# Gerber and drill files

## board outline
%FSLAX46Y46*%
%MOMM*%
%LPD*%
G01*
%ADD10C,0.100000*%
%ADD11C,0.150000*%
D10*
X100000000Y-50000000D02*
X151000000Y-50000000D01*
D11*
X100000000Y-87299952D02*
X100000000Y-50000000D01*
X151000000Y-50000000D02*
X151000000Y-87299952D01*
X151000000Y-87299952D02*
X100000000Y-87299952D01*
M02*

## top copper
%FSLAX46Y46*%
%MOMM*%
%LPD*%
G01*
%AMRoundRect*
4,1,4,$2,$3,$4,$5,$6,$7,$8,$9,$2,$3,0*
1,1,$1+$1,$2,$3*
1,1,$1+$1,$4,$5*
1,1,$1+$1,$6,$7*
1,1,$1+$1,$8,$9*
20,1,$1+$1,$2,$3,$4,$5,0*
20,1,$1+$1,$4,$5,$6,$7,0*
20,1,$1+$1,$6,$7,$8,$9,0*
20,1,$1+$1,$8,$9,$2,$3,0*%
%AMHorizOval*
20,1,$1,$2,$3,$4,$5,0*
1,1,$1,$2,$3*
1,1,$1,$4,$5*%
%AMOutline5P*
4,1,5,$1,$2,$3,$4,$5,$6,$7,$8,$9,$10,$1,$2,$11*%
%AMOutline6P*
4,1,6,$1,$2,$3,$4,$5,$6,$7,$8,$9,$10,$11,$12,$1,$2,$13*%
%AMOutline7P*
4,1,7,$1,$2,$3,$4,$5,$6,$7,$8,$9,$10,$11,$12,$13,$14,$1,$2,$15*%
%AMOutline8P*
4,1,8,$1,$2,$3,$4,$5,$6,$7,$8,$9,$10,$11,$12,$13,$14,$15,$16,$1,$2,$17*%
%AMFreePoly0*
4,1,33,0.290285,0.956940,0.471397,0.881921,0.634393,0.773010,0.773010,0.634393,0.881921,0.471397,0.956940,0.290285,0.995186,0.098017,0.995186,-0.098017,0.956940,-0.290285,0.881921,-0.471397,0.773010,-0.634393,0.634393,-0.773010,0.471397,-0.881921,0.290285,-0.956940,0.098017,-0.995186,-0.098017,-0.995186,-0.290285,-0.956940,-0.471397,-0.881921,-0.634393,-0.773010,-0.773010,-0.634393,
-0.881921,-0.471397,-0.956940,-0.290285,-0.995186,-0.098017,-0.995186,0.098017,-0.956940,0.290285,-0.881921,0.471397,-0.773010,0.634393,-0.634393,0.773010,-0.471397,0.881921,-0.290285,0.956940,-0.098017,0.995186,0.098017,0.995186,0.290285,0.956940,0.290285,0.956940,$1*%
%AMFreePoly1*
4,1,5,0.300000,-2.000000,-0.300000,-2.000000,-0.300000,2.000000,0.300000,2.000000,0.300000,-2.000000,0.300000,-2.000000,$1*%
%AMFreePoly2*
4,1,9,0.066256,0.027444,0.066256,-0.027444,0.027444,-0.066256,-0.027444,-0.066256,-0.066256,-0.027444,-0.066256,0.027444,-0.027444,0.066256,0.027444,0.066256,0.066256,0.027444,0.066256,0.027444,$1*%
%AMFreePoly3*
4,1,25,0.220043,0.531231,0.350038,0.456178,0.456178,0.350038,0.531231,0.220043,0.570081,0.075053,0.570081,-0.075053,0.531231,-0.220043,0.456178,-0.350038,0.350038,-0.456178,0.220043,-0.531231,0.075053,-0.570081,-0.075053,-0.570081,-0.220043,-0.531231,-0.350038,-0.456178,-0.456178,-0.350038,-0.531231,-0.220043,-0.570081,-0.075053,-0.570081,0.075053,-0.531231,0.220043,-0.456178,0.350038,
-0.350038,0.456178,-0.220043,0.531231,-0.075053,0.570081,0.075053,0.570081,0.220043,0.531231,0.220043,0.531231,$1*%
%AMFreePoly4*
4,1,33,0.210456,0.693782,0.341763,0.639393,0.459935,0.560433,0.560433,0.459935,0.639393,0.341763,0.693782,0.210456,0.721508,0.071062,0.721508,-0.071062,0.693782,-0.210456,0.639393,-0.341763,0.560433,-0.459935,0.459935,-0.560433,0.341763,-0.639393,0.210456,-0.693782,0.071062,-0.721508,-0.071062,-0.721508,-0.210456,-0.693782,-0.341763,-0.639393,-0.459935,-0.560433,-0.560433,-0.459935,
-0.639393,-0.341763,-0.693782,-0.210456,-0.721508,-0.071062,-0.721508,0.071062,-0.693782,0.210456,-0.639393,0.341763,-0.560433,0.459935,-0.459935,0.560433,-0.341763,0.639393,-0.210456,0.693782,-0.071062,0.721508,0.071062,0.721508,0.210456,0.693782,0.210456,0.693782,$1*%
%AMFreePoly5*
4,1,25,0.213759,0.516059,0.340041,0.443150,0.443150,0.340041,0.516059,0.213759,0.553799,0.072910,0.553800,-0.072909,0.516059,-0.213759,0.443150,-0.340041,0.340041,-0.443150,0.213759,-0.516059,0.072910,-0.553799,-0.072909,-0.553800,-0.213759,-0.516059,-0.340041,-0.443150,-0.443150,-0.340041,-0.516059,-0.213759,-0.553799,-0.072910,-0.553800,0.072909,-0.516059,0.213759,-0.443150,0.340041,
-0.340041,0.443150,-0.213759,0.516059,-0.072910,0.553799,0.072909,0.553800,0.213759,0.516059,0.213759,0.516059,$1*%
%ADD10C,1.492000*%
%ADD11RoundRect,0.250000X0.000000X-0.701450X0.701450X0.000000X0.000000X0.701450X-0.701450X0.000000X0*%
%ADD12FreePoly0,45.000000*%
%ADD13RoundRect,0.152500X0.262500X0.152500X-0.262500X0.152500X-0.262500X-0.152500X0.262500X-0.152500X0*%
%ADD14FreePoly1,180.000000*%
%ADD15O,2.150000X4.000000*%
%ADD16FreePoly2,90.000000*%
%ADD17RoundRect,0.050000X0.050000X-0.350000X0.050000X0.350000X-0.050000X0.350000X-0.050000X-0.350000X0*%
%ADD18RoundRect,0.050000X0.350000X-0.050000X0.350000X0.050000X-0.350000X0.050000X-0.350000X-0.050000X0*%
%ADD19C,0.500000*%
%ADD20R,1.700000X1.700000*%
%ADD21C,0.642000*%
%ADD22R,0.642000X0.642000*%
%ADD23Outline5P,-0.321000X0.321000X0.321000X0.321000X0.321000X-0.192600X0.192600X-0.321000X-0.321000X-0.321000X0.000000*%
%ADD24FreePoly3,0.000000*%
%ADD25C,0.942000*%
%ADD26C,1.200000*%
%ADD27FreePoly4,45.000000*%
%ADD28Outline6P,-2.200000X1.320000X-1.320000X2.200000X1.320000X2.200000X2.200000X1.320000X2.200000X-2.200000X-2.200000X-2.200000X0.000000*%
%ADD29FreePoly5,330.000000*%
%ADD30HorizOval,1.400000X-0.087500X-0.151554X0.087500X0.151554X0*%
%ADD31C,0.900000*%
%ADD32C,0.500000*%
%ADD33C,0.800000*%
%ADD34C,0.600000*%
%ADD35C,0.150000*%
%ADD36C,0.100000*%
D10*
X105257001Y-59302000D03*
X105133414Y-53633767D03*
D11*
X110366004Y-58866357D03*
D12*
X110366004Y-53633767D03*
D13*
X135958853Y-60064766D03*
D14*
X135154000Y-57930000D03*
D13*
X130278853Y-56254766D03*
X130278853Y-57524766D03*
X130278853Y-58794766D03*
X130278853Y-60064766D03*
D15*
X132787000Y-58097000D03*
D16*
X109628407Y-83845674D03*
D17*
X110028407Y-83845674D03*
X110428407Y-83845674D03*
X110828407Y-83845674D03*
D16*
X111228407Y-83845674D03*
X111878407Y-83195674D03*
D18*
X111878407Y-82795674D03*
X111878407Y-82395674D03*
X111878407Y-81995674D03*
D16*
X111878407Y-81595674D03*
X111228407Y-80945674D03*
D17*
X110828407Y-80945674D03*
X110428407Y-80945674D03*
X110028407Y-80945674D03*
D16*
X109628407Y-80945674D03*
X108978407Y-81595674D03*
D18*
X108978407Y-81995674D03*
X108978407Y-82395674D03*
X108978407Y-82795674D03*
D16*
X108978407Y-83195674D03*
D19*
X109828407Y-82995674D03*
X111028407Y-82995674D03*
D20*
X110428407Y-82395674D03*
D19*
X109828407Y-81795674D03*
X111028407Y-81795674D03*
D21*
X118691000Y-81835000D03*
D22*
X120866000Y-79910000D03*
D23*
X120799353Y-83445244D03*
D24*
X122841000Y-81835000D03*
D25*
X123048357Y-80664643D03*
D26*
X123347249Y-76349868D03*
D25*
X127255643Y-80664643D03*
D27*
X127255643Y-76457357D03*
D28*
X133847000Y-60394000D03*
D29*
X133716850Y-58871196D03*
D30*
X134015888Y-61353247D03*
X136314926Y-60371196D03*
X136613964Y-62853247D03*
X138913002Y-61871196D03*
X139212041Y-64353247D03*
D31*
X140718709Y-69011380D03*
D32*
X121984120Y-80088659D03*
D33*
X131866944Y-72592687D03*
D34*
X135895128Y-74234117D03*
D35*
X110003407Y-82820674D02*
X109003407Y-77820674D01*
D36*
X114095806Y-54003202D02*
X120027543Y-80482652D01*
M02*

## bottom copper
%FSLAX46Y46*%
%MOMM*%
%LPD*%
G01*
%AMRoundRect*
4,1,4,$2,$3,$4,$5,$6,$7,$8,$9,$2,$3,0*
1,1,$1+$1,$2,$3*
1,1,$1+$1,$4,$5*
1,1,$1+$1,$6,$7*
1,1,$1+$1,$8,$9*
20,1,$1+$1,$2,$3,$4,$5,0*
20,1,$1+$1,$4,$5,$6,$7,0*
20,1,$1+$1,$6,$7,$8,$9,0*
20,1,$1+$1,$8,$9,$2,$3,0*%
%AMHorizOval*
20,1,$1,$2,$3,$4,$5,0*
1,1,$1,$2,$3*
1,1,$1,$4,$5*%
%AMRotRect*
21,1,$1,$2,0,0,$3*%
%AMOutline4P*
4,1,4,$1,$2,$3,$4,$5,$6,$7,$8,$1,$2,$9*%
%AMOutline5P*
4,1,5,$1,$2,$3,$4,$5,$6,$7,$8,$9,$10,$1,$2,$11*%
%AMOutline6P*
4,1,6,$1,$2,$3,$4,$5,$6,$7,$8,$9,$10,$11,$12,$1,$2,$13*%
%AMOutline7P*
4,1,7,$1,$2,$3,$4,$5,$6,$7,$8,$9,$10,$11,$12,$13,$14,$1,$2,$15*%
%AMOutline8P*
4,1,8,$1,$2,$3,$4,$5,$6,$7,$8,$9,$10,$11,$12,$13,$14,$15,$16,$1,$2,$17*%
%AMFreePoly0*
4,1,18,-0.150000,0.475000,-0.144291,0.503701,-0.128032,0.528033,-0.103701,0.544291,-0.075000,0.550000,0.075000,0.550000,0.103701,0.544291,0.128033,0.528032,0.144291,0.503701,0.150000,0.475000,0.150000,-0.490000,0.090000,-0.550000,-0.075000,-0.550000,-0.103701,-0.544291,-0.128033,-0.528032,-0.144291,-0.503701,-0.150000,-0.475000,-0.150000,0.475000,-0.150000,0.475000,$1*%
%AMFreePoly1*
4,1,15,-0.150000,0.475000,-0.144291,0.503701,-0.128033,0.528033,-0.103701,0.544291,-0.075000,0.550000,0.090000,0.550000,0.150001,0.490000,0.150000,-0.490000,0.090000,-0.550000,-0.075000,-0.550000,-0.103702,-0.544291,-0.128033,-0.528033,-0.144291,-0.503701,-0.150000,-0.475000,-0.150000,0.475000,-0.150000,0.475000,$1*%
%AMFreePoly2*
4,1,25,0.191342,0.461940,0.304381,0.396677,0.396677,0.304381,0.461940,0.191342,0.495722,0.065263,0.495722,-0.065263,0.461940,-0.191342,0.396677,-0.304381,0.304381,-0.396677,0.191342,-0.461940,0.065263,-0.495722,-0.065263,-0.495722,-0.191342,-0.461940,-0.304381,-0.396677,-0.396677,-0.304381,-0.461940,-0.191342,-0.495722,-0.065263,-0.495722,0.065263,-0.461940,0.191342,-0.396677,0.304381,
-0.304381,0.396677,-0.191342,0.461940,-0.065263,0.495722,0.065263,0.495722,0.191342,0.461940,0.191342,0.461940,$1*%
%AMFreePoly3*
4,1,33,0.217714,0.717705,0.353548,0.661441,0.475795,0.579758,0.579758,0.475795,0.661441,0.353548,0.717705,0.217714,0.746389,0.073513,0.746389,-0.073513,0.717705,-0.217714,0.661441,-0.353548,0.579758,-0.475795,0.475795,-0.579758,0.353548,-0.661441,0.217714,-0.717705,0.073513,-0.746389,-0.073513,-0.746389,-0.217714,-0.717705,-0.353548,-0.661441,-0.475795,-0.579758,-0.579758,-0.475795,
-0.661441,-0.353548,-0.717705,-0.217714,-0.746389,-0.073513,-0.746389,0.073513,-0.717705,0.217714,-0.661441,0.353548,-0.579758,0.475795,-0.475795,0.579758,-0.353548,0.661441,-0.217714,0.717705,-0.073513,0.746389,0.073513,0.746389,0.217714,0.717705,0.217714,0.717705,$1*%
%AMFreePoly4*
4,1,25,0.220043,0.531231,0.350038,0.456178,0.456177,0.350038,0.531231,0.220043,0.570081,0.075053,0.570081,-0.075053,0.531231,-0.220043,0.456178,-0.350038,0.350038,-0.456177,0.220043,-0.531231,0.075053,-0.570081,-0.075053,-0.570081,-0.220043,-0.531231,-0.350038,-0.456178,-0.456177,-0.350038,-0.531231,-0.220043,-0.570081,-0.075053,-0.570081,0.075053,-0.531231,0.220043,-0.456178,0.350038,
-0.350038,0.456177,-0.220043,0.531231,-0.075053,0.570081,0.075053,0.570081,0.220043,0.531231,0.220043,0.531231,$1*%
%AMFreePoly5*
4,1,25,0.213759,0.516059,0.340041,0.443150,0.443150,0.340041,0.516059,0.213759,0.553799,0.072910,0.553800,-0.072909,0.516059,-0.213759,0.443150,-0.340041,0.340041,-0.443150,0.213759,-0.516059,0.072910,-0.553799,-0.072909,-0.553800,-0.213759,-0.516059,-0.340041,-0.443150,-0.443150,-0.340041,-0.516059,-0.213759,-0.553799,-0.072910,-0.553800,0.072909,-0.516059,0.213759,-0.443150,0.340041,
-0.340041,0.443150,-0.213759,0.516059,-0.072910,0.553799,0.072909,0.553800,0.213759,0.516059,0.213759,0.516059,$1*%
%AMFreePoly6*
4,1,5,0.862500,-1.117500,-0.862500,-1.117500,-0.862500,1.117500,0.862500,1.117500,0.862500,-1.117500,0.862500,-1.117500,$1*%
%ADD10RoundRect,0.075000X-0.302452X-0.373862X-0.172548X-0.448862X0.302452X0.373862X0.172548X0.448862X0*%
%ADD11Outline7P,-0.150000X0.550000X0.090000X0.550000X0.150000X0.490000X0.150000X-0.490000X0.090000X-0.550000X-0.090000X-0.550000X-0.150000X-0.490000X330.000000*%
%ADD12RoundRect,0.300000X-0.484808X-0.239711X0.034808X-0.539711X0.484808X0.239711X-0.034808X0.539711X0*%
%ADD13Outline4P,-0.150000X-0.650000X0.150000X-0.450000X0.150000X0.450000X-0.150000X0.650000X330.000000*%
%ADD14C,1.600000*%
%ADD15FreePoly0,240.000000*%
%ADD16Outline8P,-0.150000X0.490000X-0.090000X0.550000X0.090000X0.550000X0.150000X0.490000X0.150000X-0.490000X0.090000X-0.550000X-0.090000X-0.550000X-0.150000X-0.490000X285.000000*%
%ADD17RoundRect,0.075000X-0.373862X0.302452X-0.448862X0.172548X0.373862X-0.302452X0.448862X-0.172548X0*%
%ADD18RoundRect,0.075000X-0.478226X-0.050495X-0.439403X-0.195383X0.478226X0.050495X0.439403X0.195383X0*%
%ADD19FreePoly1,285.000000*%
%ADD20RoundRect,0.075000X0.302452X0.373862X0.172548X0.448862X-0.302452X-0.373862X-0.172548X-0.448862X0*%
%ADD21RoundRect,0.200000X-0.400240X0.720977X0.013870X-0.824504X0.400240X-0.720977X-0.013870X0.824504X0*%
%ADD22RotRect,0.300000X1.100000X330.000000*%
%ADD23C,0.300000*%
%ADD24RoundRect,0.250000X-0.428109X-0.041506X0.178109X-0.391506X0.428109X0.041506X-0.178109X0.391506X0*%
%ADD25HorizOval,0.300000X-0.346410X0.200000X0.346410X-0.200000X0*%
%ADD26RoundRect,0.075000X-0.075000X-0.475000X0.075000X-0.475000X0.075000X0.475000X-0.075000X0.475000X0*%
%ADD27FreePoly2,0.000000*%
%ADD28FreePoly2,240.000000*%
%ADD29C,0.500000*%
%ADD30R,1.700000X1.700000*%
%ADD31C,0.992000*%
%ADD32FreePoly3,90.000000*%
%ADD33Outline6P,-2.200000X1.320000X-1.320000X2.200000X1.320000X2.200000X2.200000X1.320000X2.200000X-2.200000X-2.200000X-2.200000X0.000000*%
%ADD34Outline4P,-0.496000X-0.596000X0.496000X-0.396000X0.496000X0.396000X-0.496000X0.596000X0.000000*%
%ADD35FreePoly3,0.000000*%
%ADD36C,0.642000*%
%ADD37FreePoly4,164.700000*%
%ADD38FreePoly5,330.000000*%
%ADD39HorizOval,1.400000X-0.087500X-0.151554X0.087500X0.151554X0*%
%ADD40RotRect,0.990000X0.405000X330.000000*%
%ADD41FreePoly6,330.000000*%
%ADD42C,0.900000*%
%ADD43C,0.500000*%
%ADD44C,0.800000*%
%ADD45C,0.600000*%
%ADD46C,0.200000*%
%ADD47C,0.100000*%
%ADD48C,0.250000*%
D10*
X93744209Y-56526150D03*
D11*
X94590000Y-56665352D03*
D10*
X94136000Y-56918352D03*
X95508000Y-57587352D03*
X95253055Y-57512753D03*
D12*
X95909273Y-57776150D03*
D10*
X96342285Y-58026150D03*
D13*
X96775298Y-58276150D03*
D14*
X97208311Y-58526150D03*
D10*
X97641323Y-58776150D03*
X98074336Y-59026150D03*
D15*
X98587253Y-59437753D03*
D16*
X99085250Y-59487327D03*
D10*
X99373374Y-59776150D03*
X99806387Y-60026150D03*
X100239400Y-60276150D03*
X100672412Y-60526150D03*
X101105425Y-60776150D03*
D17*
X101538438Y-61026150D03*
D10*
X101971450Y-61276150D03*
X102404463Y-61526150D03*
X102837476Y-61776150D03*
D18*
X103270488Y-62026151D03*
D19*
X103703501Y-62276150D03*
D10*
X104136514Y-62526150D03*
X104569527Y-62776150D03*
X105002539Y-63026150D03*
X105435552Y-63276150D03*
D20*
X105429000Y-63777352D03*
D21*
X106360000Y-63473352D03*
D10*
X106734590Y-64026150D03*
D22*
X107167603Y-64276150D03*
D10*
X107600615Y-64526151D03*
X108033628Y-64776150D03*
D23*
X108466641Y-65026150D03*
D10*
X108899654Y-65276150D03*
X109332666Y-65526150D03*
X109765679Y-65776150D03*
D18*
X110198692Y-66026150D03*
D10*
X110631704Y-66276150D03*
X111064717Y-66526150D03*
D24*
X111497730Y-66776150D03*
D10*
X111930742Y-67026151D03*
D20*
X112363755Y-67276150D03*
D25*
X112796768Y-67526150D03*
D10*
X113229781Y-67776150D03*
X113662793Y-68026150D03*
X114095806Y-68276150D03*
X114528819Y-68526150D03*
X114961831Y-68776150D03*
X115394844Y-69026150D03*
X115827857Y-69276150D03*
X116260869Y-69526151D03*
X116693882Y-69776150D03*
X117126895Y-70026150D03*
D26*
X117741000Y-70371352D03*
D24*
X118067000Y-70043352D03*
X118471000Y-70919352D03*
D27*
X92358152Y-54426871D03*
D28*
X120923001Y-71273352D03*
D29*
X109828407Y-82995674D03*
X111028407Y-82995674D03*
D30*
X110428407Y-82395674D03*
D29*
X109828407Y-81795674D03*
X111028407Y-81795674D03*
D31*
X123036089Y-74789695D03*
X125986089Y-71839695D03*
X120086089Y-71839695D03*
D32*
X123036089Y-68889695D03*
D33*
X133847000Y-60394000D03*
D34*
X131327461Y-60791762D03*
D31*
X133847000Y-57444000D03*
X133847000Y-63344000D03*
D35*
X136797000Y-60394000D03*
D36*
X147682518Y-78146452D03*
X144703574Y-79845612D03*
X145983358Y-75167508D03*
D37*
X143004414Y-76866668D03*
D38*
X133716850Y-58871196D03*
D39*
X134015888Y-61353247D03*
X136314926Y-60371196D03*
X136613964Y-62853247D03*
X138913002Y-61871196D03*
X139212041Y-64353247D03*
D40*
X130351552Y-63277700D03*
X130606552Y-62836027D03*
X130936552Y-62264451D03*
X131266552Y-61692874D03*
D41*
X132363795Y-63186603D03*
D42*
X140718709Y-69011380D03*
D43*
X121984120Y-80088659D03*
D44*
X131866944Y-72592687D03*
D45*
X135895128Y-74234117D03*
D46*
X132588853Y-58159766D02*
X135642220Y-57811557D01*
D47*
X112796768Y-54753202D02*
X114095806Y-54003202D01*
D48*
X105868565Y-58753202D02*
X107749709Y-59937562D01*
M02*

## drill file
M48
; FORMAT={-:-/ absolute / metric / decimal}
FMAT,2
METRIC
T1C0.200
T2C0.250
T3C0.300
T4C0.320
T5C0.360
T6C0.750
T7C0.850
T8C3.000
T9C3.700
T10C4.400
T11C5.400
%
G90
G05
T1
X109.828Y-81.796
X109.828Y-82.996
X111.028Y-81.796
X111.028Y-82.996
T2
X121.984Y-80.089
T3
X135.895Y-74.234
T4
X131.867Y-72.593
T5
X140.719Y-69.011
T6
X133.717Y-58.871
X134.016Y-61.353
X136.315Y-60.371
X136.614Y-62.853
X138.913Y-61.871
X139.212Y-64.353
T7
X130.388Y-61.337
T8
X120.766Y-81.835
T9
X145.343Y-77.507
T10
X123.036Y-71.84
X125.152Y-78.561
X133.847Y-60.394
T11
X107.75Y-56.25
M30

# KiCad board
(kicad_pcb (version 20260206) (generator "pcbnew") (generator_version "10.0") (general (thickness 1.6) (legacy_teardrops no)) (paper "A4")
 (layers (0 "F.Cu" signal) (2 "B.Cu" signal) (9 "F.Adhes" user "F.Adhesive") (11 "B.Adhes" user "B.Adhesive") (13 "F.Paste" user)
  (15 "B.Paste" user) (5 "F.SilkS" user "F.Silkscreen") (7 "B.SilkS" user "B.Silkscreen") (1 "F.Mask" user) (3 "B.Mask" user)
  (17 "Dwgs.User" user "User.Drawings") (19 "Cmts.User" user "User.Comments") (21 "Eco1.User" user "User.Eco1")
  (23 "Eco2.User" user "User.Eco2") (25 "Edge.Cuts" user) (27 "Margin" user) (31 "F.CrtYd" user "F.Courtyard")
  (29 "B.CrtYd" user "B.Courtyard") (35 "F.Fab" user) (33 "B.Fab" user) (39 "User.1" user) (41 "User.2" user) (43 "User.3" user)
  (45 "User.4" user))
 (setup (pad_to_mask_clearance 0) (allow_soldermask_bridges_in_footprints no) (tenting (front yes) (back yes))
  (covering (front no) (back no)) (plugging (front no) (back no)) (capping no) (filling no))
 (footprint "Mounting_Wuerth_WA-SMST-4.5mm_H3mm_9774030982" (layer "F.Cu") (at 107.749709 56.250062 45)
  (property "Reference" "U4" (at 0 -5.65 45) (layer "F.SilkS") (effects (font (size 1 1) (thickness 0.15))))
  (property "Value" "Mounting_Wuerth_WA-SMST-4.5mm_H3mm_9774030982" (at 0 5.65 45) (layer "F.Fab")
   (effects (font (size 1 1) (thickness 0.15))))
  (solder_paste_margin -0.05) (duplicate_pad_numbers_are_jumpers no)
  (pad "" smd custom (at -2.607456 -2.607456 15) (size 0.9475 0.9475) (layers) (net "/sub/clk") (clearance 0.1) (zone_connect 0)
   (options (clearance outline) (anchor circle)) (primitives))
  (pad "" smd custom (at -2.222894 2.681511 90) (size 0.8 0.8) (layers "F.Paste") (options (clearance outline) (anchor circle)) (primitives))
  (pad "" np_thru_hole circle (at 0 0 90) (size 5.4 5.4) (drill 5.4) (layers "*.Cu" "*.Mask") (solder_mask_margin 0.05) (clearance 0.2))
  (pad "" smd custom (at 2.607456 -2.607456 135) (size 0.9475 0.9475) (drill (offset -0.2 -0.1)) (layers "F.Paste") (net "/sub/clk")
   (thermal_bridge_angle 30) (options (clearance outline) (anchor circle)) (primitives))
  (pad "" smd custom (at 2.607456 2.607456 45) (size 0.9475 0.9475) (layers "F.Paste") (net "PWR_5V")
   (options (clearance outline) (anchor circle)) (primitives))
  (pad "1" smd circle (at -3.920657 0.395435 45) (size 1.492 1.492) (layers "F.Cu"))
  (pad "1" smd circle (at 0 -3.7 45) (size 1.492 1.492) (layers "F.Cu") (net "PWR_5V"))
  (pad "A1" smd roundrect (at 0 3.7 45) (size 1.492 1.492) (layers "F.Cu") (roundrect_rratio 0.16756))
  (pad "1" smd custom (at 3.7 0 45) (size 2 2) (layers "F.Cu" "F.Mask") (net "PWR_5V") (clearance 0.1) (thermal_gap 0.3)
   (options (clearance outline) (anchor circle)) (primitives)))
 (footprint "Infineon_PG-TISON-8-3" (layer "F.Cu") (at 133.118853 58.159766 180)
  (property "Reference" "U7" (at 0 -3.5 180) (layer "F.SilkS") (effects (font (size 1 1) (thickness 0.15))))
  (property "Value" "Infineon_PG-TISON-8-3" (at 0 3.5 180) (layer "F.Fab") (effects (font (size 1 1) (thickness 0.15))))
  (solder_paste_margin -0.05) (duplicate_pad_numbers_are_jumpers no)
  (pad "" smd rect (at -2.84 -0.635 180) (size 0.73 0.51) (layers "F.Paste"))
  (pad "" smd rect (at -2.84 0.635 180) (size 0.73 0.51) (layers "B.Mask" "F.SilkS") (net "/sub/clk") (clearance 0.1) (thermal_gap 0.3))
  (pad "" smd rect (at -2.84 1.905 180) (size 0.73 0.51) (layers "F.Paste") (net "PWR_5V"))
  (pad "" smd rect (at -1.82 -0.64 180) (size 0.9 0.5) (layers "F.Paste"))
  (pad "" smd rect (at -1.82 0.06 180) (size 0.9 0.5) (layers "F.Paste") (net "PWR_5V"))
  (pad "" smd rect (at -1.647147 0.676766 180) (size 1.2 1.5) (layers "F.Paste") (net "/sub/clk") (clearance 0.1) (thermal_gap 0.5))
  (pad "" smd rect (at -1.82 1.46 180) (size 0.9 0.5) (layers "F.Paste") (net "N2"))
  (pad "" smd rect (at -1.545 -1.6 225) (size 0.35 0.6) (layers "F.Paste") (solder_mask_margin 0.05) (solder_paste_margin -0.03)
   (thermal_bridge_width 0.4))
  (pad "" smd rect (at -0.169147 -1.557234 180) (size 0.75 0.75) (layers "F.Paste") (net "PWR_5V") (thermal_bridge_angle 45))
  (pad "" smd rect (at 0 -0.475 225) (size 0.75 0.75) (layers "F.Paste") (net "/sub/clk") (solder_mask_margin 0.05) (clearance 0.1))
  (pad "" smd rect (at 0 0.475 180) (size 0.75 0.75) (layers "F.Paste") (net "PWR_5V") (clearance 0.1))
  (pad "" smd rect (at 0 1.425 180) (size 0.75 0.75) (layers "F.Paste") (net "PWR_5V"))
  (pad "" smd rect (at 1.025 -1.425 180) (size 0.75 0.75) (layers "B.Mask" "F.Paste" "Dwgs.User") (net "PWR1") (clearance 0.1)
   (zone_connect 2))
  (pad "" smd rect (at 1.025 -0.475 180) (size 0.75 0.75) (layers "F.Paste") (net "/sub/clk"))
  (pad "" smd rect (at 1.025 0.475 180) (size 0.75 0.75) (layers "F.Paste") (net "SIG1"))
  (pad "" smd rect (at 1.025 1.425 180) (size 0.75 0.75) (layers "F.Paste"))
  (pad "1" smd roundrect (at -2.84 -1.905 180) (size 0.83 0.61) (layers "F.Cu" "F.Mask" "F.Paste") (roundrect_rratio 0.25) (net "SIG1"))
  (pad "2" smd custom (at -2.035147 0.229766 180) (size 0.6 4) (layers "F.Cu" "F.Mask") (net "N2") (clearance 0.1) (thermal_bridge_angle 45)
   (options (clearance outline) (anchor rect)) (primitives))
  (pad "3" smd roundrect (at 2.84 1.905 180) (size 0.83 0.61) (layers "F.Cu" "F.Mask" "F.Paste") (roundrect_rratio 0.25))
  (pad "4" smd roundrect (at 2.84 0.635 180) (size 0.83 0.61) (layers "F.Cu" "F.Mask" "F.Paste") (roundrect_rratio 0.25) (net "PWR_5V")
   (clearance 0.1))
  (pad "5" smd roundrect (at 2.84 -0.635 180) (size 0.83 0.61) (layers "F.Cu" "F.Mask" "F.Paste") (roundrect_rratio 0.25) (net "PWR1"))
  (pad "6" smd roundrect (at 2.84 -1.905 180) (size 0.83 0.61) (layers "F.Cu" "F.Mask" "F.Paste") (roundrect_rratio 0.25) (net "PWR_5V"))
  (pad "7" smd oval (at 0.331853 0.062766 180) (size 2.15 4) (layers "*.Mask" "F.Cu")))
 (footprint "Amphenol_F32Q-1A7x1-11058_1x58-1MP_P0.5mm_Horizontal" (layer "B.Cu") (at 107.535071 61.139676 -30)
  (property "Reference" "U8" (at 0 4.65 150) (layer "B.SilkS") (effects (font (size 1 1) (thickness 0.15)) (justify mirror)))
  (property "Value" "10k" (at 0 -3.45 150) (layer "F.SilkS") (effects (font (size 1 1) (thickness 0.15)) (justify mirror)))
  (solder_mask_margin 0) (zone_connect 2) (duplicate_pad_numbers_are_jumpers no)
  (pad "1" smd roundrect (at -14.25 2.9 330) (size 0.3 1.1) (layers "B.Cu" "B.Mask" "B.Paste") (roundrect_rratio 0.25))
  (pad "A1" smd roundrect (at -13.447922 2.597657 330) (size 0.3 1.1) (layers "B.Cu" "B.Mask" "B.Paste") (roundrect_rratio 0)
   (chamfer_ratio 0.2) (chamfer top_right bottom_left bottom_right) (thermal_bridge_angle 30))
  (pad "3" smd roundrect (at -13.714598 3.043762 330) (size 0.3 1.1) (layers "B.Cu" "B.Mask" "B.Paste") (roundrect_rratio 0.25))
  (pad "4" smd roundrect (at -12.191911 2.937133 330) (size 0.3 1.1) (layers "B.Cu" "B.Mask" "B.Paste") (roundrect_rratio 0.25) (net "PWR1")
   (thermal_bridge_width 0.4))
  (pad "5" smd roundrect (at -12.25 2.9 330) (size 0.3 1.1) (drill (offset -0.2 0.1)) (layers "B.Cu" "B.Mask" "B.Paste")
   (roundrect_rratio 0.25) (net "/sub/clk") (zone_connect 2))
  (pad "6" smd roundrect (at -11.749999 2.9 330) (size 1.2 1.5) (layers "B.Cu" "B.Mask" "B.Paste") (roundrect_rratio 0.25) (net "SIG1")
   (clearance 0.1) (zone_connect 2))
  (pad "7" smd roundrect (at -11.25 2.9 330) (size 0.3 1.1) (layers "B.Cu" "B.Mask" "B.Paste") (roundrect_rratio 0.25) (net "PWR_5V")
   (solder_paste_margin -0.03) (clearance 0.2) (zone_connect 1) (thermal_bridge_width 0.4))
  (pad "8" smd trapezoid (at -10.75 2.9 330) (size 0.3 1.1) (rect_delta 0.2 0) (layers "B.Cu" "B.Mask" "B.Paste") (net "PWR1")
   (clearance 0.1) (zone_connect 0))
  (pad "9" smd circle (at -10.249999 2.9 285) (size 1.6 1.6) (layers "B.Cu" "B.Mask" "B.Paste") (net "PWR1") (zone_connect 0))
  (pad "10" smd roundrect (at -9.75 2.9 330) (size 0.3 1.1) (layers "B.Cu" "B.Mask" "B.Paste") (roundrect_rratio 0.25))
  (pad "A1" smd roundrect (at -9.25 2.9 330) (size 0.3 1.1) (layers "B.Cu" "B.Mask" "B.Paste") (roundrect_rratio 0.25) (thermal_gap 0.5))
  (pad "12" smd roundrect (at -8.75 2.9 240) (size 0.3 1.1) (drill (offset 0.1 -0.15)) (layers "B.Cu" "B.Mask" "B.Paste")
   (roundrect_rratio 0.25) (chamfer_ratio 0.2) (chamfer bottom_right) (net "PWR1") (solder_paste_margin -0.03) (clearance 0.1))
  (pad "1" smd roundrect (at -8.25 2.9 285) (size 0.3 1.1) (drill (offset 0 -0.15)) (layers "*.Mask" "B.Cu" "B.SilkS" "B.Paste" "Dwgs.User")
   (roundrect_rratio 0) (chamfer_ratio 0.2) (chamfer top_left top_right bottom_left bottom_right) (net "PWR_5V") (thermal_gap 0.5))
  (pad "14" smd roundrect (at -7.75 2.9 330) (size 0.3 1.1) (layers "B.Cu" "B.Mask" "B.Paste") (roundrect_rratio 0.25))
  (pad "15" smd roundrect (at -7.25 2.9 330) (size 0.3 1.1) (layers "B.Cu" "B.Mask" "B.Paste") (roundrect_rratio 0.25) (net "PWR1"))
  (pad "16" smd roundrect (at -6.749999 2.9 330) (size 0.3 1.1) (layers "B.Cu" "B.Mask" "B.Paste") (roundrect_rratio 0.25))
  (pad "17" smd roundrect (at -6.25 2.9 330) (size 0.3 1.1) (layers "B.Cu" "B.Mask" "B.Paste") (roundrect_rratio 0.25) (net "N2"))
  (pad "18" smd roundrect (at -5.75 2.9 330) (size 0.3 1.1) (layers "B.Cu" "B.Mask" "B.Paste") (roundrect_rratio 0.25) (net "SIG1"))
  (pad "19" smd roundrect (at -5.25 2.9 240) (size 0.3 1.1) (layers "B.Cu" "B.Mask" "B.Paste") (roundrect_rratio 0.25) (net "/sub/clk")
   (clearance 0.35))
  (pad "20" smd roundrect (at -4.75 2.9 330) (size 0.3 1.1) (layers "B.Cu" "B.Mask" "B.Paste") (roundrect_rratio 0.25) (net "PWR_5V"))
  (pad "21" smd roundrect (at -4.25 2.9 330) (size 0.3 1.1) (layers "B.Cu" "B.Mask" "B.Paste") (roundrect_rratio 0.25) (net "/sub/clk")
   (clearance 0.1))
  (pad "22" smd roundrect (at -3.75 2.9 330) (size 0.3 1.1) (layers "B.Cu" "B.Mask" "B.Paste") (roundrect_rratio 0.25) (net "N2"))
  (pad "2" smd roundrect (at -3.25 2.900001 285) (size 0.3 1.1) (layers "B.Cu" "B.Mask" "B.Paste") (roundrect_rratio 0.25) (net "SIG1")
   (solder_paste_margin -0.03) (zone_connect 2))
  (pad "24" smd roundrect (at -2.75 2.9 285) (size 0.3 1.1) (layers "B.Cu" "B.Mask" "B.Paste" "Dwgs.User" "Eco1.User")
   (roundrect_rratio 0.25) (chamfer_ratio 0.2) (chamfer top_right bottom_right) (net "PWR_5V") (zone_connect 2))
  (pad "25" smd roundrect (at -2.25 2.9 330) (size 0.3 1.1) (layers "B.Cu" "B.Mask" "B.Paste") (roundrect_rratio 0.25))
  (pad "26" smd roundrect (at -1.749999 2.9 330) (size 0.3 1.1) (layers "B.Cu" "B.Mask" "B.Paste") (roundrect_rratio 0.25))
  (pad "27" smd roundrect (at -1.25 2.9 330) (size 0.3 1.1) (layers "B.Cu" "B.Mask" "B.Paste") (roundrect_rratio 0.25) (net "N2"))
  (pad "28" smd roundrect (at -0.75 2.9 330) (size 0.3 1.1) (layers "B.Cu" "B.Mask" "B.Paste") (roundrect_rratio 0.25) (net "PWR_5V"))
  (pad "29" smd roundrect (at -0.505073 3.33733 150) (size 0.3 1.1) (layers "B.Cu" "B.Mask" "B.Paste") (roundrect_rratio 0.25) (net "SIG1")
   (solder_paste_margin -0.03) (zone_connect 0))
  (pad "30" smd roundrect (at 0.149197 2.608558 285) (size 2 0.8) (layers "B.Cu" "B.Mask" "B.Paste") (roundrect_rratio 0.25) (clearance 0.1)
   (thermal_gap 0.5))
  (pad "31" smd roundrect (at 0.75 2.9 330) (size 0.3 1.1) (layers "B.Cu" "B.Mask" "B.Paste") (roundrect_rratio 0.25))
  (pad "32" smd rect (at 1.25 2.9 330) (size 0.3 1.1) (layers "*.Mask" "B.Cu" "B.Paste") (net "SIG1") (clearance 0.2)
   (thermal_bridge_width 0.25))
  (pad "33" smd roundrect (at 1.75 2.900001 330) (size 0.3 1.1) (layers "B.Cu" "B.Mask" "B.Paste") (roundrect_rratio 0.25) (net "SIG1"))
  (pad "34" smd roundrect (at 2.25 2.9 330) (size 0.3 1.1) (layers "B.Cu" "B.Mask" "B.Paste") (roundrect_rratio 0.25) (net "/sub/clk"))
  (pad "35" smd circle (at 2.75 2.9 330) (size 0.3 0.3) (layers "B.Cu" "B.Mask" "B.Paste") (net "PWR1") (solder_mask_margin 0.05)
   (clearance 0.35) (zone_connect 0) (thermal_gap 0.3))
  (pad "36" smd roundrect (at 3.250001 2.9 330) (size 0.3 1.1) (layers "B.Cu" "B.Mask" "B.Paste") (roundrect_rratio 0.25) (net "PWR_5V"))
  (pad "EP" smd roundrect (at 3.75 2.9 330) (size 0.3 1.1) (layers "B.Cu" "B.Mask" "B.Paste") (roundrect_rratio 0.25))
  (pad "38" smd roundrect (at 4.25 2.9 330) (size 0.3 1.1) (layers "B.Cu" "B.Mask" "B.Paste") (roundrect_rratio 0.25))
  (pad "2" smd roundrect (at 4.75 2.9 285) (size 0.3 1.1) (layers "B.Cu" "B.Mask" "B.Paste") (roundrect_rratio 0.25)
   (solder_paste_margin -0.03) (clearance 0.2))
  (pad "40" smd roundrect (at 5.25 2.9 330) (size 0.3 1.1) (layers "B.Cu" "B.Mask" "B.Paste") (roundrect_rratio 0.25) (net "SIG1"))
  (pad "41" smd roundrect (at 5.75 2.9 330) (size 0.3 1.1) (layers "B.Cu" "B.Mask" "B.Paste") (roundrect_rratio 0.25))
  (pad "42" smd roundrect (at 6.25 2.9 330) (size 1.2 1) (layers "B.Cu" "B.Mask" "B.Paste") (roundrect_rratio 0.25) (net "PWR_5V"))
  (pad "43" smd roundrect (at 6.75 2.900001 330) (size 0.3 1.1) (layers "B.Cu" "B.Mask" "B.Paste") (roundrect_rratio 0.25) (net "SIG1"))
  (pad "1" smd roundrect (at 7.25 2.9 150) (size 0.3 1.1) (layers "B.Cu" "B.Mask" "B.Paste") (roundrect_rratio 0.25) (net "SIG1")
   (solder_paste_margin -0.03))
  (pad "45" smd oval (at 7.75 2.9 240) (size 0.3 1.1) (layers "B.Cu" "B.Mask" "Eco1.User") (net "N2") (thermal_bridge_angle 30))
  (pad "46" smd roundrect (at 8.250001 2.9 330) (size 0.3 1.1) (layers "B.Cu" "B.Mask" "B.Paste") (roundrect_rratio 0.25) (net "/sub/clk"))
  (pad "47" smd roundrect (at 8.75 2.9 330) (size 0.3 1.1) (layers "B.Cu" "B.Mask" "B.Paste") (roundrect_rratio 0.25) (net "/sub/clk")
   (clearance 0.35))
  (pad "48" smd roundrect (at 9.25 2.9 330) (size 0.3 1.1) (layers "B.Cu" "B.Mask" "B.Paste") (roundrect_rratio 0.25) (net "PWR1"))
  (pad "49" smd roundrect (at 9.75 2.9 330) (size 0.3 1.1) (layers "B.Cu" "B.Mask" "B.Paste") (roundrect_rratio 0.25) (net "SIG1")
   (clearance 0.1))
  (pad "50" smd roundrect (at 10.25 2.9 330) (size 0.3 1.1) (layers "B.Cu" "B.Mask" "B.Paste") (roundrect_rratio 0.25) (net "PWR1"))
  (pad "1" smd roundrect (at 10.75 2.9 330) (size 0.3 1.1) (layers "*.Mask" "B.Cu" "B.Paste" "Dwgs.User") (roundrect_rratio 0.25)
   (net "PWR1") (solder_paste_margin -0.03) (clearance 0.1))
  (pad "52" smd roundrect (at 11.25 2.9 330) (size 0.3 1.1) (layers "B.Cu" "B.Mask" "B.Paste") (roundrect_rratio 0.25))
  (pad "53" smd roundrect (at 11.75 2.900001 330) (size 0.3 1.1) (layers "B.Cu" "B.Mask" "B.Paste") (roundrect_rratio 0.25))
  (pad "54" smd roundrect (at 12.25 2.9 330) (size 0.3 1.1) (layers "B.Cu" "B.Mask" "B.Paste") (roundrect_rratio 0.25) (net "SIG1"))
  (pad "55" smd roundrect (at 12.75 2.9 330) (size 0.3 1.1) (layers "B.Cu" "B.Mask" "B.Paste") (roundrect_rratio 0.25)
   (solder_mask_margin 0.05) (zone_connect 0))
  (pad "1" smd roundrect (at 13.454432 2.891901) (size 0.3 1.1) (layers "B.Cu" "B.Mask" "B.Paste") (roundrect_rratio 0.25) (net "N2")
   (clearance 0.2) (zone_connect 0) (thermal_bridge_width 0.4))
  (pad "57" smd roundrect (at 13.572756 2.444845 330) (size 1.2 1) (layers "B.Cu" "B.Mask" "B.Paste") (roundrect_rratio 0.25)
   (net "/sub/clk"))
  (pad "58" smd roundrect (at 14.36063 3.001483 330) (size 1.2 1) (layers "B.Cu" "B.Mask" "B.Paste") (roundrect_rratio 0.25)
   (zone_connect 1))
  (pad "MP" smd custom (at -16.5 1.775) (size 1 1) (layers "B.Cu" "B.Mask" "B.Paste") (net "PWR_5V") (thermal_bridge_angle 90)
   (thermal_gap 0.5) (options (clearance outline) (anchor circle)) (primitives))
  (pad "MP" smd custom (at 16.661125 2.082056 240) (size 1 1) (layers "B.Cu" "B.Mask" "B.Paste") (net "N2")
   (options (clearance outline) (anchor circle)) (primitives)))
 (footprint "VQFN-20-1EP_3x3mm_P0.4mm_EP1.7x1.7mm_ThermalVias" (layer "F.Cu") (at 110.428407 82.395674 90)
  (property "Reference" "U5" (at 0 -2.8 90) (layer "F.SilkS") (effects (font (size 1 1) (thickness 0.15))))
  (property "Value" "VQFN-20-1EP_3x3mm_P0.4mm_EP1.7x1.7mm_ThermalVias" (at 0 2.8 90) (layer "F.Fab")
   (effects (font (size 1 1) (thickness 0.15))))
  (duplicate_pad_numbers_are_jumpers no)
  (pad "" smd roundrect (at -0.425 -0.425 90) (size 0.74 0.74) (layers "F.Paste") (roundrect_rratio 0.25) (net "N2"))
  (pad "" smd roundrect (at -0.425 0.425 90) (size 0.74 0.74) (layers "F.Paste") (roundrect_rratio 0.25) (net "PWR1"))
  (pad "" smd roundrect (at 0.425 -0.425 90) (size 0.74 0.74) (layers "F.Paste") (roundrect_rratio 0.25) (clearance 0.1))
  (pad "" smd roundrect (at 0.425 0.425 90) (size 0.74 0.74) (layers "F.Paste") (roundrect_rratio 0.25) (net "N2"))
  (pad "1" smd custom (at -1.45 -0.8 90) (size 0.143431 0.143431) (layers "F.Cu" "F.Mask" "F.Paste")
   (options (clearance outline) (anchor circle)) (primitives))
  (pad "2" smd roundrect (at -1.45 -0.4 90) (size 0.8 0.2) (layers "F.Cu" "F.Mask" "F.Paste") (roundrect_rratio 0.25) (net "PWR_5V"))
  (pad "3" smd roundrect (at -1.45 0 90) (size 0.8 0.2) (layers "F.Cu" "F.Mask" "F.Paste") (roundrect_rratio 0.25) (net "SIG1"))
  (pad "4" smd roundrect (at -1.45 0.4 90) (size 0.8 0.2) (layers "F.Cu" "F.Mask" "F.Paste") (roundrect_rratio 0.25) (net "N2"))
  (pad "5" smd custom (at -1.45 0.8 90) (size 0.143431 0.143431) (layers "F.Cu" "F.Mask" "F.Paste") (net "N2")
   (options (clearance outline) (anchor circle)) (primitives))
  (pad "6" smd custom (at -0.8 1.45 90) (size 0.143431 0.143431) (layers "F.Cu" "F.Mask" "F.Paste") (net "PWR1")
   (options (clearance outline) (anchor circle)) (primitives))
  (pad "7" smd roundrect (at -0.4 1.45 90) (size 0.2 0.8) (layers "F.Cu" "F.Mask" "F.Paste") (roundrect_rratio 0.25) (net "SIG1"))
  (pad "8" smd roundrect (at 0 1.45 90) (size 0.2 0.8) (layers "F.Cu" "F.Mask" "F.Paste") (roundrect_rratio 0.25))
  (pad "9" smd roundrect (at 0.4 1.45 90) (size 0.2 0.8) (layers "F.Cu" "F.Mask" "F.Paste") (roundrect_rratio 0.25))
  (pad "10" smd custom (at 0.8 1.45 90) (size 0.143431 0.143431) (layers "F.Cu" "F.Mask" "F.Paste") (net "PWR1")
   (options (clearance outline) (anchor circle)) (primitives))
  (pad "11" smd custom (at 1.45 0.8 90) (size 0.143431 0.143431) (layers "F.Cu" "F.Mask" "F.Paste") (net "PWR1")
   (options (clearance outline) (anchor circle)) (primitives))
  (pad "12" smd roundrect (at 1.45 0.4 90) (size 0.8 0.2) (layers "F.Cu" "F.Mask" "F.Paste") (roundrect_rratio 0.25))
  (pad "13" smd roundrect (at 1.45 0 90) (size 0.8 0.2) (layers "F.Cu" "F.Mask" "F.Paste") (roundrect_rratio 0.25) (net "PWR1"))
  (pad "14" smd roundrect (at 1.45 -0.4 90) (size 0.8 0.2) (layers "F.Cu" "F.Mask" "F.Paste") (roundrect_rratio 0.25) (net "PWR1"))
  (pad "15" smd custom (at 1.45 -0.8 90) (size 0.143431 0.143431) (layers "F.Cu" "F.Mask" "F.Paste") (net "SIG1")
   (options (clearance outline) (anchor circle)) (primitives))
  (pad "16" smd custom (at 0.8 -1.45 90) (size 0.143431 0.143431) (layers "F.Cu" "F.Mask" "F.Paste") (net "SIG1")
   (options (clearance outline) (anchor circle)) (primitives))
  (pad "17" smd roundrect (at 0.4 -1.45 90) (size 0.2 0.8) (layers "F.Cu" "F.Mask" "F.Paste") (roundrect_rratio 0.25) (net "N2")
   (clearance 0.35))
  (pad "18" smd roundrect (at 0 -1.45 90) (size 0.2 0.8) (layers "F.Cu" "F.Mask" "F.Paste") (roundrect_rratio 0.25) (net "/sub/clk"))
  (pad "19" smd roundrect (at -0.4 -1.45 90) (size 0.2 0.8) (layers "F.Cu" "F.Mask" "F.Paste") (roundrect_rratio 0.25))
  (pad "20" smd custom (at -0.8 -1.45 90) (size 0.143431 0.143431) (layers "F.Cu" "F.Mask" "F.Paste") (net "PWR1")
   (options (clearance outline) (anchor circle)) (primitives))
  (pad "21" thru_hole circle (at -0.6 -0.6 90) (size 0.5 0.5) (drill 0.2) (layers "*.Cu") (remove_unused_layers no) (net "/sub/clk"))
  (pad "21" thru_hole circle (at -0.6 0.6 90) (size 0.5 0.5) (drill 0.2) (layers "*.Cu") (remove_unused_layers no) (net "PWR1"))
  (pad "21" smd rect (at 0 0 90) (size 1.7 1.7) (layers "F.Cu" "F.Mask") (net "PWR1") (zone_connect 2))
  (pad "21" smd rect (at 0 0 90) (size 1.7 1.7) (layers "B.Cu") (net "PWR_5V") (zone_connect 2))
  (pad "21" thru_hole circle (at 0.6 -0.6 90) (size 0.5 0.5) (drill 0.2) (layers "*.Cu") (remove_unused_layers no) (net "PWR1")
   (clearance 0.35))
  (pad "21" thru_hole circle (at 0.6 0.6 90) (size 0.5 0.5) (drill 0.2) (layers "*.Cu") (remove_unused_layers no) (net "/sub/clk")
   (clearance 0.35)))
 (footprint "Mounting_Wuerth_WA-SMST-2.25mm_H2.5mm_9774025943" (layer "F.Cu") (at 120.766 81.835)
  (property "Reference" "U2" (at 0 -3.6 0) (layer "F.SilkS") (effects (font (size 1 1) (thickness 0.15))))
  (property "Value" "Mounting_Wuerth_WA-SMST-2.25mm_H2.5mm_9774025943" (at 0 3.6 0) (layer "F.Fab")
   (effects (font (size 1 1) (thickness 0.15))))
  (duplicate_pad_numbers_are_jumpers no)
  (pad "" smd custom (at -1.453104 -1.453104) (size 0.505 0.505) (layers "F.Paste") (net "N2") (options (clearance outline) (anchor circle))
   (primitives))
  (pad "" smd custom (at -1.453104 1.453104 330) (size 1.6 1.6) (layers "F.Paste") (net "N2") (zone_connect 0)
   (options (clearance outline) (anchor circle)) (primitives))
  (pad "" np_thru_hole circle (at 0 0) (size 3 3) (drill 3) (layers "*.Cu" "*.Mask"))
  (pad "" smd custom (at 1.106353 -0.954756 180) (size 0.505 0.505) (drill (offset -0.2 0)) (layers "F.Paste" "Dwgs.User" "Eco1.User")
   (clearance 0.1) (zone_connect 0) (thermal_bridge_width 0.4) (options (clearance outline) (anchor circle)) (primitives))
  (pad "" smd custom (at 1.453104 1.453104) (size 0.505 0.505) (layers "F.Paste") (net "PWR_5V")
   (options (clearance outline) (anchor circle)) (primitives))
  (pad "1" smd circle (at -2.075 0) (size 0.642 0.642) (layers "F.Cu") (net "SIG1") (solder_paste_margin -0.03) (zone_connect 2)
   (thermal_gap 0.3))
  (pad "1" smd rect (at 0 -2.075) (size 0.642 0.642) (drill (offset 0.1 0.15)) (layers "F.Cu" "F.SilkS") (solder_mask_margin 0)
   (clearance 0.2) (zone_connect 0))
  (pad "1" smd roundrect (at 0.033353 1.610244) (size 0.642 0.642) (layers "F.Cu") (roundrect_rratio 0) (chamfer_ratio 0.2)
   (chamfer bottom_right) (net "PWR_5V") (solder_mask_margin 0.05) (clearance 0.1) (zone_connect 1))
  (pad "1" smd custom (at 2.075 0) (size 1.15 1.15) (layers "F.Cu" "F.Mask") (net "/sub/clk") (options (clearance outline) (anchor circle))
   (primitives)))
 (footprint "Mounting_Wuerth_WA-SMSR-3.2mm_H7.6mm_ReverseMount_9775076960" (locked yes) (layer "F.Cu") (at 125.152 78.561 45)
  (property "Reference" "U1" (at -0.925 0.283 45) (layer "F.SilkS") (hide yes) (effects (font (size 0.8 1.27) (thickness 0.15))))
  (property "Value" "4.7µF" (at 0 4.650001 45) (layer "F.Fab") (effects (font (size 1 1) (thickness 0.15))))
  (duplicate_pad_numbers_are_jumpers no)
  (pad "" smd custom (at -2.094804 -2.094804 45) (size 0.6725 0.6725) (layers "F.Paste") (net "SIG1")
   (options (clearance outline) (anchor circle)) (primitives))
  (pad "" smd custom (at -2.094804 2.094804 45) (size 0.6725 0.6725) (layers "F.Paste") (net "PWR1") (clearance 0.1)
   (options (clearance outline) (anchor circle)) (primitives))
  (pad "" np_thru_hole circle (at 0 0 45) (size 4.4 4.4) (drill 4.4 (offset 0 -0.1)) (layers "*.Cu" "*.Mask") (clearance 0.35)
   (zone_connect 1))
  (pad "" smd custom (at 2.094804 -2.094804 45) (size 0.6725 0.6725) (layers "F.Paste") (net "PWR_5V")
   (options (clearance outline) (anchor circle)) (primitives))
  (pad "" smd custom (at 2.094804 2.094804 45) (size 0.6725 0.6725) (layers "F.Paste") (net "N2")
   (options (clearance outline) (anchor circle)) (primitives))
  (pad "1" smd circle (at -2.975 0 45) (size 0.942 0.942) (layers "F.Cu") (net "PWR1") (clearance 0.1))
  (pad "1" smd circle (at 0.287355 -2.839658 90) (size 1.2 1.2) (layers "F.Cu") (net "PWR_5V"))
  (pad "1" smd circle (at 0 2.975 45) (size 0.942 0.942) (layers "F.Cu") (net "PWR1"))
  (pad "1" smd custom (at 2.975 0 45) (size 1.45 1.45) (layers "F.Cu" "F.Mask") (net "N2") (options (clearance outline) (anchor circle))
   (primitives)))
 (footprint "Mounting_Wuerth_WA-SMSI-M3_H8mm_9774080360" (layer "B.Cu") (at 123.036089 71.839695 90)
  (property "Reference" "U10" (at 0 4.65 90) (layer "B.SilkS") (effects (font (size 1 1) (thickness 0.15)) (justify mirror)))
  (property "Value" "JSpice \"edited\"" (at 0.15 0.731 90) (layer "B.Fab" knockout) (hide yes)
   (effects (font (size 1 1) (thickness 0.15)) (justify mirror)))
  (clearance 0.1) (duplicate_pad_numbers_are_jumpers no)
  (pad "" smd custom (at -2.057681 2.057681 90) (size 0.55 0.55) (layers "B.Paste") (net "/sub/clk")
   (options (clearance outline) (anchor circle)) (primitives))
  (pad "" smd custom (at -2.057681 -2.057681 90) (size 0.55 0.55) (layers "B.Paste") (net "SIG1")
   (options (clearance outline) (anchor circle)) (primitives))
  (pad "" np_thru_hole oval (at 0 0 90) (size 1.6 0.8) (drill 4.4) (layers "*.Cu" "B.Mask" "Eco1.User") (thermal_bridge_width 0.25))
  (pad "" smd custom (at 1.779305 2.300911 90) (size 0.55 0.55) (layers "B.Paste") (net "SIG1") (solder_paste_margin -0.03) (zone_connect 2)
   (options (clearance outline) (anchor circle)) (primitives))
  (pad "" smd custom (at 2.057681 -2.057681 90) (size 0.55 0.55) (layers "B.Paste") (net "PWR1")
   (options (clearance outline) (anchor circle)) (primitives))
  (pad "1" smd circle (at -2.95 0 90) (size 0.992 0.992) (layers "B.Cu") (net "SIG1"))
  (pad "1" smd circle (at 0 2.95 90) (size 0.992 0.992) (layers "B.Cu") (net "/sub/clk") (clearance 0.1))
  (pad "1" smd circle (at 0 -2.95 90) (size 0.992 0.992) (layers "B.Cu" "Dwgs.User") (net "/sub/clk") (clearance 0.35)
   (thermal_bridge_angle 90))
  (pad "1" smd custom (at 2.95 0 90) (size 1.5 1.5) (layers "B.Cu" "B.Mask") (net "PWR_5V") (options (clearance outline) (anchor circle))
   (primitives)))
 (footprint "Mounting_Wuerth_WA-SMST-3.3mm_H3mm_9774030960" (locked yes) (layer "B.Cu") (at 133.847 60.394)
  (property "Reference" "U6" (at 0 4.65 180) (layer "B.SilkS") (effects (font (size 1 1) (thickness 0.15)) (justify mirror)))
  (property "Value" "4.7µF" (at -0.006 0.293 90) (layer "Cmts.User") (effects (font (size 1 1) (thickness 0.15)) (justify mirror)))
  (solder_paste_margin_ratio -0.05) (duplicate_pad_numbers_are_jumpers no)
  (pad "" smd custom (at -2.331539 -1.937238) (size 0.55 0.55) (layers "B.Paste") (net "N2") (solder_paste_margin -0.03) (thermal_gap 0.5)
   (options (clearance outline) (anchor circle)) (primitives))
  (pad "" smd custom (at -2.057681 2.057681) (size 0.55 0.55) (layers "B.Paste") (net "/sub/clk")
   (options (clearance outline) (anchor circle)) (primitives))
  (pad "" np_thru_hole roundrect (at 0 0) (size 4.4 4.4) (drill 4.4) (layers "*.Cu" "*.Mask") (roundrect_rratio 0) (chamfer_ratio 0.2)
   (chamfer top_left top_right) (clearance 0.2))
  (pad "" smd custom (at 2.057681 -2.057681) (size 1.2 1.2) (layers "B.Paste") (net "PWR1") (zone_connect 2) (thermal_bridge_angle 90)
   (options (clearance outline) (anchor circle)) (primitives))
  (pad "" smd custom (at 2.057681 2.057681) (size 0.55 0.55) (layers "B.Paste") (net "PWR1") (thermal_bridge_width 0.4)
   (thermal_bridge_angle 30) (options (clearance outline) (anchor circle)) (primitives))
  (pad "1" smd trapezoid (at -2.519539 0.397762) (size 0.992 0.992) (rect_delta 0.2 0) (layers "B.Cu" "B.SilkS" "Dwgs.User") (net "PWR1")
   (solder_mask_margin 0) (clearance 0.35) (thermal_bridge_width 0.4) (thermal_bridge_angle 30))
  (pad "1" smd circle (at 0 -2.95) (size 0.992 0.992) (layers "B.Cu"))
  (pad "1" smd circle (at 0 2.95) (size 0.992 0.992) (layers "B.Cu") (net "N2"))
  (pad "1" smd custom (at 2.95 0) (size 1.5 1.5) (layers "B.Cu" "B.Mask") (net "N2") (thermal_bridge_width 0.25) (thermal_bridge_angle 90)
   (thermal_gap 0.3) (options (clearance outline) (anchor circle)) (primitives)))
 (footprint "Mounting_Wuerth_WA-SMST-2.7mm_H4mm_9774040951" (layer "B.Cu") (at 145.343466 77.50656 164.7)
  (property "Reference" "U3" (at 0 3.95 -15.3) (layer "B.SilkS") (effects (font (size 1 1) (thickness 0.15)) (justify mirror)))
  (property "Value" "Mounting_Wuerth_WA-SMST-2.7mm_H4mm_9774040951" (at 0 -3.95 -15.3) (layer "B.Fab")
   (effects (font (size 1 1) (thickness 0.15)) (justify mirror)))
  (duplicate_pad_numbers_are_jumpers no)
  (pad "" smd custom (at -1.704127 -1.704127 164.7) (size 0.51 0.51) (layers "B.Paste") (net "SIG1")
   (options (clearance outline) (anchor circle)) (primitives))
  (pad "" smd custom (at -1.704127 1.704127 164.7) (size 0.51 0.51) (layers "B.Paste") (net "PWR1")
   (options (clearance outline) (anchor circle)) (primitives))
  (pad "" np_thru_hole circle (at 0 0 164.7) (size 3.7 3.7) (drill 3.7) (layers "*.Cu" "*.Mask"))
  (pad "" smd custom (at 1.704127 -1.704127 164.7) (size 0.51 0.51) (layers "B.Paste") (options (clearance outline) (anchor circle))
   (primitives))
  (pad "" smd custom (at 1.704127 1.704127 164.7) (size 0.51 0.51) (layers "B.Paste") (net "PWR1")
   (options (clearance outline) (anchor circle)) (primitives))
  (pad "1" smd circle (at -2.425 0 164.7) (size 0.642 0.642) (layers "B.Cu") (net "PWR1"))
  (pad "1" smd circle (at 0 -2.425 164.7) (size 0.642 0.642) (layers "B.Cu"))
  (pad "1" smd circle (at 0 2.425 164.7) (size 0.642 0.642) (layers "B.Cu") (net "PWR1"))
  (pad "1" smd custom (at 2.425 0 164.7) (size 1.15 1.15) (layers "B.Cu" "B.Mask") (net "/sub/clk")
   (options (clearance outline) (anchor circle)) (primitives)))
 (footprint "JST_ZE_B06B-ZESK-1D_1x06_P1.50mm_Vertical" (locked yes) (layer "B.Cu") (at 133.71685 58.871196 -30)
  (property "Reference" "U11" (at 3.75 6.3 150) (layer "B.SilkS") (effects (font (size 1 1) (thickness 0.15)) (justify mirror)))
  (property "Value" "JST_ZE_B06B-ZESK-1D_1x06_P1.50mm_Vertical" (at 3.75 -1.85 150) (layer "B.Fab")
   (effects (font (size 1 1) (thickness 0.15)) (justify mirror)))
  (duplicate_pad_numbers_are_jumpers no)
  (pad "" np_thru_hole circle (at -1.65 3.8 330) (size 0.85 0.85) (drill 0.85) (layers "*.Cu" "*.Mask"))
  (pad "1" thru_hole custom (at 0 0 330) (size 1.117157 1.117157) (drill 0.75) (layers "*.Cu" "*.Mask") (remove_unused_layers no)
   (options (clearance outline) (anchor circle)) (primitives))
  (pad "2" thru_hole oval (at 1.5 2 330) (size 1.4 1.75) (drill 0.75) (layers "*.Cu" "*.Mask") (remove_unused_layers no))
  (pad "3" thru_hole oval (at 3 0 330) (size 1.4 1.75) (drill 0.75) (layers "*.Cu" "*.Mask") (remove_unused_layers no) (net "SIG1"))
  (pad "4" thru_hole oval (at 4.5 2 330) (size 1.4 1.75) (drill 0.75) (layers "*.Cu" "*.Mask") (remove_unused_layers no))
  (pad "5" thru_hole oval (at 6 0 330) (size 1.4 1.75) (drill 0.75) (layers "*.Cu" "*.Mask") (remove_unused_layers no))
  (pad "6" thru_hole oval (at 7.500001 2 330) (size 1.4 1.75) (drill 0.75) (layers "*.Cu" "*.Mask") (remove_unused_layers no)
   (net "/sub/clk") (clearance 0.1)))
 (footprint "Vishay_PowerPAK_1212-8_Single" (layer "B.Cu") (at 132.014298 63.267739 -30)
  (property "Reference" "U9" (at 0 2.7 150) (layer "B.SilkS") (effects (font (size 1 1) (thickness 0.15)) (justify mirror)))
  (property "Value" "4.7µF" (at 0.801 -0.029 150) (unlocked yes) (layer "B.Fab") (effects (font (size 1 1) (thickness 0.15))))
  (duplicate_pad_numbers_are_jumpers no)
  (pad "1" smd rect (at -1.435 0.99 330) (size 0.99 0.405) (drill (offset 0 -0.15)) (layers "B.Cu" "B.Mask" "B.Paste" "Eco1.User")
   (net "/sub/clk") (solder_paste_margin -0.03))
  (pad "2" smd rect (at -1.435 0.329999 330) (size 0.99 0.405) (layers "B.Cu" "B.Mask" "B.Paste") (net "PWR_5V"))
  (pad "3" smd rect (at -1.434999 -0.33 330) (size 0.99 0.405) (layers "B.Cu" "B.Mask" "B.Paste") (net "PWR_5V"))
  (pad "4" smd rect (at -1.435 -0.99 330) (size 0.99 0.405) (layers "B.Cu" "B.Mask" "B.Paste") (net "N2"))
  (pad "5" smd custom (at 0.462105 -0.345015 330) (size 1.725 2.235) (drill (offset -0.2 0.1)) (layers "B.Cu" "B.Mask" "B.Paste") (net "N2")
   (zone_connect 2) (thermal_bridge_angle 45) (options (clearance outline) (anchor rect)) (primitives)))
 (gr_line (start 100 50) (end 151 50) (stroke (width 0.1) (type default)) (layer "Edge.Cuts"))
 (gr_line (start 100 87.299952) (end 100 50) (stroke (width 0.15) (type default)) (layer "Edge.Cuts"))
 (gr_line (start 151 50) (end 151 87.299952) (stroke (width 0.15) (type default)) (layer "Edge.Cuts"))
 (gr_line (start 151 87.299952) (end 100 87.299952) (stroke (width 0.15) (type default)) (layer "Edge.Cuts"))
 (segment (start 110.003407 82.820674) (end 109.003407 77.820674) (width 0.15) (layer "F.Cu") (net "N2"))
 (via (at 140.718709 69.01138) (size 0.9) (drill 0.36) (layers "F.Cu" "B.Cu") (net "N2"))
 (via (at 121.98412 80.088659) (size 0.5) (drill 0.25) (layers "F.Cu" "B.Cu") (locked yes) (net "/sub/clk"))
 (segment (start 132.588853 58.159766) (end 135.64222 57.811557) (width 0.2) (layer "B.Cu") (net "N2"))
 (segment (start 112.796768 54.753202) (end 114.095806 54.003202) (width 0.1) (layer "B.Cu") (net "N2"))
 (via (at 131.866944 72.592687) (size 0.8) (drill 0.32) (layers "F.Cu" "B.Cu") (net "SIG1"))
 (via (at 135.895128 74.234117) (size 0.6) (drill 0.3) (layers "F.Cu" "B.Cu") (locked yes) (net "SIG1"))
 (segment (start 105.868565 58.753202) (end 107.749709 59.937562) (width 0.25) (layer "B.Cu") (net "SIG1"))
 (segment (start 114.095806 54.003202) (end 120.027543 80.482652) (width 0.1) (layer "F.Cu") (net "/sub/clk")))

